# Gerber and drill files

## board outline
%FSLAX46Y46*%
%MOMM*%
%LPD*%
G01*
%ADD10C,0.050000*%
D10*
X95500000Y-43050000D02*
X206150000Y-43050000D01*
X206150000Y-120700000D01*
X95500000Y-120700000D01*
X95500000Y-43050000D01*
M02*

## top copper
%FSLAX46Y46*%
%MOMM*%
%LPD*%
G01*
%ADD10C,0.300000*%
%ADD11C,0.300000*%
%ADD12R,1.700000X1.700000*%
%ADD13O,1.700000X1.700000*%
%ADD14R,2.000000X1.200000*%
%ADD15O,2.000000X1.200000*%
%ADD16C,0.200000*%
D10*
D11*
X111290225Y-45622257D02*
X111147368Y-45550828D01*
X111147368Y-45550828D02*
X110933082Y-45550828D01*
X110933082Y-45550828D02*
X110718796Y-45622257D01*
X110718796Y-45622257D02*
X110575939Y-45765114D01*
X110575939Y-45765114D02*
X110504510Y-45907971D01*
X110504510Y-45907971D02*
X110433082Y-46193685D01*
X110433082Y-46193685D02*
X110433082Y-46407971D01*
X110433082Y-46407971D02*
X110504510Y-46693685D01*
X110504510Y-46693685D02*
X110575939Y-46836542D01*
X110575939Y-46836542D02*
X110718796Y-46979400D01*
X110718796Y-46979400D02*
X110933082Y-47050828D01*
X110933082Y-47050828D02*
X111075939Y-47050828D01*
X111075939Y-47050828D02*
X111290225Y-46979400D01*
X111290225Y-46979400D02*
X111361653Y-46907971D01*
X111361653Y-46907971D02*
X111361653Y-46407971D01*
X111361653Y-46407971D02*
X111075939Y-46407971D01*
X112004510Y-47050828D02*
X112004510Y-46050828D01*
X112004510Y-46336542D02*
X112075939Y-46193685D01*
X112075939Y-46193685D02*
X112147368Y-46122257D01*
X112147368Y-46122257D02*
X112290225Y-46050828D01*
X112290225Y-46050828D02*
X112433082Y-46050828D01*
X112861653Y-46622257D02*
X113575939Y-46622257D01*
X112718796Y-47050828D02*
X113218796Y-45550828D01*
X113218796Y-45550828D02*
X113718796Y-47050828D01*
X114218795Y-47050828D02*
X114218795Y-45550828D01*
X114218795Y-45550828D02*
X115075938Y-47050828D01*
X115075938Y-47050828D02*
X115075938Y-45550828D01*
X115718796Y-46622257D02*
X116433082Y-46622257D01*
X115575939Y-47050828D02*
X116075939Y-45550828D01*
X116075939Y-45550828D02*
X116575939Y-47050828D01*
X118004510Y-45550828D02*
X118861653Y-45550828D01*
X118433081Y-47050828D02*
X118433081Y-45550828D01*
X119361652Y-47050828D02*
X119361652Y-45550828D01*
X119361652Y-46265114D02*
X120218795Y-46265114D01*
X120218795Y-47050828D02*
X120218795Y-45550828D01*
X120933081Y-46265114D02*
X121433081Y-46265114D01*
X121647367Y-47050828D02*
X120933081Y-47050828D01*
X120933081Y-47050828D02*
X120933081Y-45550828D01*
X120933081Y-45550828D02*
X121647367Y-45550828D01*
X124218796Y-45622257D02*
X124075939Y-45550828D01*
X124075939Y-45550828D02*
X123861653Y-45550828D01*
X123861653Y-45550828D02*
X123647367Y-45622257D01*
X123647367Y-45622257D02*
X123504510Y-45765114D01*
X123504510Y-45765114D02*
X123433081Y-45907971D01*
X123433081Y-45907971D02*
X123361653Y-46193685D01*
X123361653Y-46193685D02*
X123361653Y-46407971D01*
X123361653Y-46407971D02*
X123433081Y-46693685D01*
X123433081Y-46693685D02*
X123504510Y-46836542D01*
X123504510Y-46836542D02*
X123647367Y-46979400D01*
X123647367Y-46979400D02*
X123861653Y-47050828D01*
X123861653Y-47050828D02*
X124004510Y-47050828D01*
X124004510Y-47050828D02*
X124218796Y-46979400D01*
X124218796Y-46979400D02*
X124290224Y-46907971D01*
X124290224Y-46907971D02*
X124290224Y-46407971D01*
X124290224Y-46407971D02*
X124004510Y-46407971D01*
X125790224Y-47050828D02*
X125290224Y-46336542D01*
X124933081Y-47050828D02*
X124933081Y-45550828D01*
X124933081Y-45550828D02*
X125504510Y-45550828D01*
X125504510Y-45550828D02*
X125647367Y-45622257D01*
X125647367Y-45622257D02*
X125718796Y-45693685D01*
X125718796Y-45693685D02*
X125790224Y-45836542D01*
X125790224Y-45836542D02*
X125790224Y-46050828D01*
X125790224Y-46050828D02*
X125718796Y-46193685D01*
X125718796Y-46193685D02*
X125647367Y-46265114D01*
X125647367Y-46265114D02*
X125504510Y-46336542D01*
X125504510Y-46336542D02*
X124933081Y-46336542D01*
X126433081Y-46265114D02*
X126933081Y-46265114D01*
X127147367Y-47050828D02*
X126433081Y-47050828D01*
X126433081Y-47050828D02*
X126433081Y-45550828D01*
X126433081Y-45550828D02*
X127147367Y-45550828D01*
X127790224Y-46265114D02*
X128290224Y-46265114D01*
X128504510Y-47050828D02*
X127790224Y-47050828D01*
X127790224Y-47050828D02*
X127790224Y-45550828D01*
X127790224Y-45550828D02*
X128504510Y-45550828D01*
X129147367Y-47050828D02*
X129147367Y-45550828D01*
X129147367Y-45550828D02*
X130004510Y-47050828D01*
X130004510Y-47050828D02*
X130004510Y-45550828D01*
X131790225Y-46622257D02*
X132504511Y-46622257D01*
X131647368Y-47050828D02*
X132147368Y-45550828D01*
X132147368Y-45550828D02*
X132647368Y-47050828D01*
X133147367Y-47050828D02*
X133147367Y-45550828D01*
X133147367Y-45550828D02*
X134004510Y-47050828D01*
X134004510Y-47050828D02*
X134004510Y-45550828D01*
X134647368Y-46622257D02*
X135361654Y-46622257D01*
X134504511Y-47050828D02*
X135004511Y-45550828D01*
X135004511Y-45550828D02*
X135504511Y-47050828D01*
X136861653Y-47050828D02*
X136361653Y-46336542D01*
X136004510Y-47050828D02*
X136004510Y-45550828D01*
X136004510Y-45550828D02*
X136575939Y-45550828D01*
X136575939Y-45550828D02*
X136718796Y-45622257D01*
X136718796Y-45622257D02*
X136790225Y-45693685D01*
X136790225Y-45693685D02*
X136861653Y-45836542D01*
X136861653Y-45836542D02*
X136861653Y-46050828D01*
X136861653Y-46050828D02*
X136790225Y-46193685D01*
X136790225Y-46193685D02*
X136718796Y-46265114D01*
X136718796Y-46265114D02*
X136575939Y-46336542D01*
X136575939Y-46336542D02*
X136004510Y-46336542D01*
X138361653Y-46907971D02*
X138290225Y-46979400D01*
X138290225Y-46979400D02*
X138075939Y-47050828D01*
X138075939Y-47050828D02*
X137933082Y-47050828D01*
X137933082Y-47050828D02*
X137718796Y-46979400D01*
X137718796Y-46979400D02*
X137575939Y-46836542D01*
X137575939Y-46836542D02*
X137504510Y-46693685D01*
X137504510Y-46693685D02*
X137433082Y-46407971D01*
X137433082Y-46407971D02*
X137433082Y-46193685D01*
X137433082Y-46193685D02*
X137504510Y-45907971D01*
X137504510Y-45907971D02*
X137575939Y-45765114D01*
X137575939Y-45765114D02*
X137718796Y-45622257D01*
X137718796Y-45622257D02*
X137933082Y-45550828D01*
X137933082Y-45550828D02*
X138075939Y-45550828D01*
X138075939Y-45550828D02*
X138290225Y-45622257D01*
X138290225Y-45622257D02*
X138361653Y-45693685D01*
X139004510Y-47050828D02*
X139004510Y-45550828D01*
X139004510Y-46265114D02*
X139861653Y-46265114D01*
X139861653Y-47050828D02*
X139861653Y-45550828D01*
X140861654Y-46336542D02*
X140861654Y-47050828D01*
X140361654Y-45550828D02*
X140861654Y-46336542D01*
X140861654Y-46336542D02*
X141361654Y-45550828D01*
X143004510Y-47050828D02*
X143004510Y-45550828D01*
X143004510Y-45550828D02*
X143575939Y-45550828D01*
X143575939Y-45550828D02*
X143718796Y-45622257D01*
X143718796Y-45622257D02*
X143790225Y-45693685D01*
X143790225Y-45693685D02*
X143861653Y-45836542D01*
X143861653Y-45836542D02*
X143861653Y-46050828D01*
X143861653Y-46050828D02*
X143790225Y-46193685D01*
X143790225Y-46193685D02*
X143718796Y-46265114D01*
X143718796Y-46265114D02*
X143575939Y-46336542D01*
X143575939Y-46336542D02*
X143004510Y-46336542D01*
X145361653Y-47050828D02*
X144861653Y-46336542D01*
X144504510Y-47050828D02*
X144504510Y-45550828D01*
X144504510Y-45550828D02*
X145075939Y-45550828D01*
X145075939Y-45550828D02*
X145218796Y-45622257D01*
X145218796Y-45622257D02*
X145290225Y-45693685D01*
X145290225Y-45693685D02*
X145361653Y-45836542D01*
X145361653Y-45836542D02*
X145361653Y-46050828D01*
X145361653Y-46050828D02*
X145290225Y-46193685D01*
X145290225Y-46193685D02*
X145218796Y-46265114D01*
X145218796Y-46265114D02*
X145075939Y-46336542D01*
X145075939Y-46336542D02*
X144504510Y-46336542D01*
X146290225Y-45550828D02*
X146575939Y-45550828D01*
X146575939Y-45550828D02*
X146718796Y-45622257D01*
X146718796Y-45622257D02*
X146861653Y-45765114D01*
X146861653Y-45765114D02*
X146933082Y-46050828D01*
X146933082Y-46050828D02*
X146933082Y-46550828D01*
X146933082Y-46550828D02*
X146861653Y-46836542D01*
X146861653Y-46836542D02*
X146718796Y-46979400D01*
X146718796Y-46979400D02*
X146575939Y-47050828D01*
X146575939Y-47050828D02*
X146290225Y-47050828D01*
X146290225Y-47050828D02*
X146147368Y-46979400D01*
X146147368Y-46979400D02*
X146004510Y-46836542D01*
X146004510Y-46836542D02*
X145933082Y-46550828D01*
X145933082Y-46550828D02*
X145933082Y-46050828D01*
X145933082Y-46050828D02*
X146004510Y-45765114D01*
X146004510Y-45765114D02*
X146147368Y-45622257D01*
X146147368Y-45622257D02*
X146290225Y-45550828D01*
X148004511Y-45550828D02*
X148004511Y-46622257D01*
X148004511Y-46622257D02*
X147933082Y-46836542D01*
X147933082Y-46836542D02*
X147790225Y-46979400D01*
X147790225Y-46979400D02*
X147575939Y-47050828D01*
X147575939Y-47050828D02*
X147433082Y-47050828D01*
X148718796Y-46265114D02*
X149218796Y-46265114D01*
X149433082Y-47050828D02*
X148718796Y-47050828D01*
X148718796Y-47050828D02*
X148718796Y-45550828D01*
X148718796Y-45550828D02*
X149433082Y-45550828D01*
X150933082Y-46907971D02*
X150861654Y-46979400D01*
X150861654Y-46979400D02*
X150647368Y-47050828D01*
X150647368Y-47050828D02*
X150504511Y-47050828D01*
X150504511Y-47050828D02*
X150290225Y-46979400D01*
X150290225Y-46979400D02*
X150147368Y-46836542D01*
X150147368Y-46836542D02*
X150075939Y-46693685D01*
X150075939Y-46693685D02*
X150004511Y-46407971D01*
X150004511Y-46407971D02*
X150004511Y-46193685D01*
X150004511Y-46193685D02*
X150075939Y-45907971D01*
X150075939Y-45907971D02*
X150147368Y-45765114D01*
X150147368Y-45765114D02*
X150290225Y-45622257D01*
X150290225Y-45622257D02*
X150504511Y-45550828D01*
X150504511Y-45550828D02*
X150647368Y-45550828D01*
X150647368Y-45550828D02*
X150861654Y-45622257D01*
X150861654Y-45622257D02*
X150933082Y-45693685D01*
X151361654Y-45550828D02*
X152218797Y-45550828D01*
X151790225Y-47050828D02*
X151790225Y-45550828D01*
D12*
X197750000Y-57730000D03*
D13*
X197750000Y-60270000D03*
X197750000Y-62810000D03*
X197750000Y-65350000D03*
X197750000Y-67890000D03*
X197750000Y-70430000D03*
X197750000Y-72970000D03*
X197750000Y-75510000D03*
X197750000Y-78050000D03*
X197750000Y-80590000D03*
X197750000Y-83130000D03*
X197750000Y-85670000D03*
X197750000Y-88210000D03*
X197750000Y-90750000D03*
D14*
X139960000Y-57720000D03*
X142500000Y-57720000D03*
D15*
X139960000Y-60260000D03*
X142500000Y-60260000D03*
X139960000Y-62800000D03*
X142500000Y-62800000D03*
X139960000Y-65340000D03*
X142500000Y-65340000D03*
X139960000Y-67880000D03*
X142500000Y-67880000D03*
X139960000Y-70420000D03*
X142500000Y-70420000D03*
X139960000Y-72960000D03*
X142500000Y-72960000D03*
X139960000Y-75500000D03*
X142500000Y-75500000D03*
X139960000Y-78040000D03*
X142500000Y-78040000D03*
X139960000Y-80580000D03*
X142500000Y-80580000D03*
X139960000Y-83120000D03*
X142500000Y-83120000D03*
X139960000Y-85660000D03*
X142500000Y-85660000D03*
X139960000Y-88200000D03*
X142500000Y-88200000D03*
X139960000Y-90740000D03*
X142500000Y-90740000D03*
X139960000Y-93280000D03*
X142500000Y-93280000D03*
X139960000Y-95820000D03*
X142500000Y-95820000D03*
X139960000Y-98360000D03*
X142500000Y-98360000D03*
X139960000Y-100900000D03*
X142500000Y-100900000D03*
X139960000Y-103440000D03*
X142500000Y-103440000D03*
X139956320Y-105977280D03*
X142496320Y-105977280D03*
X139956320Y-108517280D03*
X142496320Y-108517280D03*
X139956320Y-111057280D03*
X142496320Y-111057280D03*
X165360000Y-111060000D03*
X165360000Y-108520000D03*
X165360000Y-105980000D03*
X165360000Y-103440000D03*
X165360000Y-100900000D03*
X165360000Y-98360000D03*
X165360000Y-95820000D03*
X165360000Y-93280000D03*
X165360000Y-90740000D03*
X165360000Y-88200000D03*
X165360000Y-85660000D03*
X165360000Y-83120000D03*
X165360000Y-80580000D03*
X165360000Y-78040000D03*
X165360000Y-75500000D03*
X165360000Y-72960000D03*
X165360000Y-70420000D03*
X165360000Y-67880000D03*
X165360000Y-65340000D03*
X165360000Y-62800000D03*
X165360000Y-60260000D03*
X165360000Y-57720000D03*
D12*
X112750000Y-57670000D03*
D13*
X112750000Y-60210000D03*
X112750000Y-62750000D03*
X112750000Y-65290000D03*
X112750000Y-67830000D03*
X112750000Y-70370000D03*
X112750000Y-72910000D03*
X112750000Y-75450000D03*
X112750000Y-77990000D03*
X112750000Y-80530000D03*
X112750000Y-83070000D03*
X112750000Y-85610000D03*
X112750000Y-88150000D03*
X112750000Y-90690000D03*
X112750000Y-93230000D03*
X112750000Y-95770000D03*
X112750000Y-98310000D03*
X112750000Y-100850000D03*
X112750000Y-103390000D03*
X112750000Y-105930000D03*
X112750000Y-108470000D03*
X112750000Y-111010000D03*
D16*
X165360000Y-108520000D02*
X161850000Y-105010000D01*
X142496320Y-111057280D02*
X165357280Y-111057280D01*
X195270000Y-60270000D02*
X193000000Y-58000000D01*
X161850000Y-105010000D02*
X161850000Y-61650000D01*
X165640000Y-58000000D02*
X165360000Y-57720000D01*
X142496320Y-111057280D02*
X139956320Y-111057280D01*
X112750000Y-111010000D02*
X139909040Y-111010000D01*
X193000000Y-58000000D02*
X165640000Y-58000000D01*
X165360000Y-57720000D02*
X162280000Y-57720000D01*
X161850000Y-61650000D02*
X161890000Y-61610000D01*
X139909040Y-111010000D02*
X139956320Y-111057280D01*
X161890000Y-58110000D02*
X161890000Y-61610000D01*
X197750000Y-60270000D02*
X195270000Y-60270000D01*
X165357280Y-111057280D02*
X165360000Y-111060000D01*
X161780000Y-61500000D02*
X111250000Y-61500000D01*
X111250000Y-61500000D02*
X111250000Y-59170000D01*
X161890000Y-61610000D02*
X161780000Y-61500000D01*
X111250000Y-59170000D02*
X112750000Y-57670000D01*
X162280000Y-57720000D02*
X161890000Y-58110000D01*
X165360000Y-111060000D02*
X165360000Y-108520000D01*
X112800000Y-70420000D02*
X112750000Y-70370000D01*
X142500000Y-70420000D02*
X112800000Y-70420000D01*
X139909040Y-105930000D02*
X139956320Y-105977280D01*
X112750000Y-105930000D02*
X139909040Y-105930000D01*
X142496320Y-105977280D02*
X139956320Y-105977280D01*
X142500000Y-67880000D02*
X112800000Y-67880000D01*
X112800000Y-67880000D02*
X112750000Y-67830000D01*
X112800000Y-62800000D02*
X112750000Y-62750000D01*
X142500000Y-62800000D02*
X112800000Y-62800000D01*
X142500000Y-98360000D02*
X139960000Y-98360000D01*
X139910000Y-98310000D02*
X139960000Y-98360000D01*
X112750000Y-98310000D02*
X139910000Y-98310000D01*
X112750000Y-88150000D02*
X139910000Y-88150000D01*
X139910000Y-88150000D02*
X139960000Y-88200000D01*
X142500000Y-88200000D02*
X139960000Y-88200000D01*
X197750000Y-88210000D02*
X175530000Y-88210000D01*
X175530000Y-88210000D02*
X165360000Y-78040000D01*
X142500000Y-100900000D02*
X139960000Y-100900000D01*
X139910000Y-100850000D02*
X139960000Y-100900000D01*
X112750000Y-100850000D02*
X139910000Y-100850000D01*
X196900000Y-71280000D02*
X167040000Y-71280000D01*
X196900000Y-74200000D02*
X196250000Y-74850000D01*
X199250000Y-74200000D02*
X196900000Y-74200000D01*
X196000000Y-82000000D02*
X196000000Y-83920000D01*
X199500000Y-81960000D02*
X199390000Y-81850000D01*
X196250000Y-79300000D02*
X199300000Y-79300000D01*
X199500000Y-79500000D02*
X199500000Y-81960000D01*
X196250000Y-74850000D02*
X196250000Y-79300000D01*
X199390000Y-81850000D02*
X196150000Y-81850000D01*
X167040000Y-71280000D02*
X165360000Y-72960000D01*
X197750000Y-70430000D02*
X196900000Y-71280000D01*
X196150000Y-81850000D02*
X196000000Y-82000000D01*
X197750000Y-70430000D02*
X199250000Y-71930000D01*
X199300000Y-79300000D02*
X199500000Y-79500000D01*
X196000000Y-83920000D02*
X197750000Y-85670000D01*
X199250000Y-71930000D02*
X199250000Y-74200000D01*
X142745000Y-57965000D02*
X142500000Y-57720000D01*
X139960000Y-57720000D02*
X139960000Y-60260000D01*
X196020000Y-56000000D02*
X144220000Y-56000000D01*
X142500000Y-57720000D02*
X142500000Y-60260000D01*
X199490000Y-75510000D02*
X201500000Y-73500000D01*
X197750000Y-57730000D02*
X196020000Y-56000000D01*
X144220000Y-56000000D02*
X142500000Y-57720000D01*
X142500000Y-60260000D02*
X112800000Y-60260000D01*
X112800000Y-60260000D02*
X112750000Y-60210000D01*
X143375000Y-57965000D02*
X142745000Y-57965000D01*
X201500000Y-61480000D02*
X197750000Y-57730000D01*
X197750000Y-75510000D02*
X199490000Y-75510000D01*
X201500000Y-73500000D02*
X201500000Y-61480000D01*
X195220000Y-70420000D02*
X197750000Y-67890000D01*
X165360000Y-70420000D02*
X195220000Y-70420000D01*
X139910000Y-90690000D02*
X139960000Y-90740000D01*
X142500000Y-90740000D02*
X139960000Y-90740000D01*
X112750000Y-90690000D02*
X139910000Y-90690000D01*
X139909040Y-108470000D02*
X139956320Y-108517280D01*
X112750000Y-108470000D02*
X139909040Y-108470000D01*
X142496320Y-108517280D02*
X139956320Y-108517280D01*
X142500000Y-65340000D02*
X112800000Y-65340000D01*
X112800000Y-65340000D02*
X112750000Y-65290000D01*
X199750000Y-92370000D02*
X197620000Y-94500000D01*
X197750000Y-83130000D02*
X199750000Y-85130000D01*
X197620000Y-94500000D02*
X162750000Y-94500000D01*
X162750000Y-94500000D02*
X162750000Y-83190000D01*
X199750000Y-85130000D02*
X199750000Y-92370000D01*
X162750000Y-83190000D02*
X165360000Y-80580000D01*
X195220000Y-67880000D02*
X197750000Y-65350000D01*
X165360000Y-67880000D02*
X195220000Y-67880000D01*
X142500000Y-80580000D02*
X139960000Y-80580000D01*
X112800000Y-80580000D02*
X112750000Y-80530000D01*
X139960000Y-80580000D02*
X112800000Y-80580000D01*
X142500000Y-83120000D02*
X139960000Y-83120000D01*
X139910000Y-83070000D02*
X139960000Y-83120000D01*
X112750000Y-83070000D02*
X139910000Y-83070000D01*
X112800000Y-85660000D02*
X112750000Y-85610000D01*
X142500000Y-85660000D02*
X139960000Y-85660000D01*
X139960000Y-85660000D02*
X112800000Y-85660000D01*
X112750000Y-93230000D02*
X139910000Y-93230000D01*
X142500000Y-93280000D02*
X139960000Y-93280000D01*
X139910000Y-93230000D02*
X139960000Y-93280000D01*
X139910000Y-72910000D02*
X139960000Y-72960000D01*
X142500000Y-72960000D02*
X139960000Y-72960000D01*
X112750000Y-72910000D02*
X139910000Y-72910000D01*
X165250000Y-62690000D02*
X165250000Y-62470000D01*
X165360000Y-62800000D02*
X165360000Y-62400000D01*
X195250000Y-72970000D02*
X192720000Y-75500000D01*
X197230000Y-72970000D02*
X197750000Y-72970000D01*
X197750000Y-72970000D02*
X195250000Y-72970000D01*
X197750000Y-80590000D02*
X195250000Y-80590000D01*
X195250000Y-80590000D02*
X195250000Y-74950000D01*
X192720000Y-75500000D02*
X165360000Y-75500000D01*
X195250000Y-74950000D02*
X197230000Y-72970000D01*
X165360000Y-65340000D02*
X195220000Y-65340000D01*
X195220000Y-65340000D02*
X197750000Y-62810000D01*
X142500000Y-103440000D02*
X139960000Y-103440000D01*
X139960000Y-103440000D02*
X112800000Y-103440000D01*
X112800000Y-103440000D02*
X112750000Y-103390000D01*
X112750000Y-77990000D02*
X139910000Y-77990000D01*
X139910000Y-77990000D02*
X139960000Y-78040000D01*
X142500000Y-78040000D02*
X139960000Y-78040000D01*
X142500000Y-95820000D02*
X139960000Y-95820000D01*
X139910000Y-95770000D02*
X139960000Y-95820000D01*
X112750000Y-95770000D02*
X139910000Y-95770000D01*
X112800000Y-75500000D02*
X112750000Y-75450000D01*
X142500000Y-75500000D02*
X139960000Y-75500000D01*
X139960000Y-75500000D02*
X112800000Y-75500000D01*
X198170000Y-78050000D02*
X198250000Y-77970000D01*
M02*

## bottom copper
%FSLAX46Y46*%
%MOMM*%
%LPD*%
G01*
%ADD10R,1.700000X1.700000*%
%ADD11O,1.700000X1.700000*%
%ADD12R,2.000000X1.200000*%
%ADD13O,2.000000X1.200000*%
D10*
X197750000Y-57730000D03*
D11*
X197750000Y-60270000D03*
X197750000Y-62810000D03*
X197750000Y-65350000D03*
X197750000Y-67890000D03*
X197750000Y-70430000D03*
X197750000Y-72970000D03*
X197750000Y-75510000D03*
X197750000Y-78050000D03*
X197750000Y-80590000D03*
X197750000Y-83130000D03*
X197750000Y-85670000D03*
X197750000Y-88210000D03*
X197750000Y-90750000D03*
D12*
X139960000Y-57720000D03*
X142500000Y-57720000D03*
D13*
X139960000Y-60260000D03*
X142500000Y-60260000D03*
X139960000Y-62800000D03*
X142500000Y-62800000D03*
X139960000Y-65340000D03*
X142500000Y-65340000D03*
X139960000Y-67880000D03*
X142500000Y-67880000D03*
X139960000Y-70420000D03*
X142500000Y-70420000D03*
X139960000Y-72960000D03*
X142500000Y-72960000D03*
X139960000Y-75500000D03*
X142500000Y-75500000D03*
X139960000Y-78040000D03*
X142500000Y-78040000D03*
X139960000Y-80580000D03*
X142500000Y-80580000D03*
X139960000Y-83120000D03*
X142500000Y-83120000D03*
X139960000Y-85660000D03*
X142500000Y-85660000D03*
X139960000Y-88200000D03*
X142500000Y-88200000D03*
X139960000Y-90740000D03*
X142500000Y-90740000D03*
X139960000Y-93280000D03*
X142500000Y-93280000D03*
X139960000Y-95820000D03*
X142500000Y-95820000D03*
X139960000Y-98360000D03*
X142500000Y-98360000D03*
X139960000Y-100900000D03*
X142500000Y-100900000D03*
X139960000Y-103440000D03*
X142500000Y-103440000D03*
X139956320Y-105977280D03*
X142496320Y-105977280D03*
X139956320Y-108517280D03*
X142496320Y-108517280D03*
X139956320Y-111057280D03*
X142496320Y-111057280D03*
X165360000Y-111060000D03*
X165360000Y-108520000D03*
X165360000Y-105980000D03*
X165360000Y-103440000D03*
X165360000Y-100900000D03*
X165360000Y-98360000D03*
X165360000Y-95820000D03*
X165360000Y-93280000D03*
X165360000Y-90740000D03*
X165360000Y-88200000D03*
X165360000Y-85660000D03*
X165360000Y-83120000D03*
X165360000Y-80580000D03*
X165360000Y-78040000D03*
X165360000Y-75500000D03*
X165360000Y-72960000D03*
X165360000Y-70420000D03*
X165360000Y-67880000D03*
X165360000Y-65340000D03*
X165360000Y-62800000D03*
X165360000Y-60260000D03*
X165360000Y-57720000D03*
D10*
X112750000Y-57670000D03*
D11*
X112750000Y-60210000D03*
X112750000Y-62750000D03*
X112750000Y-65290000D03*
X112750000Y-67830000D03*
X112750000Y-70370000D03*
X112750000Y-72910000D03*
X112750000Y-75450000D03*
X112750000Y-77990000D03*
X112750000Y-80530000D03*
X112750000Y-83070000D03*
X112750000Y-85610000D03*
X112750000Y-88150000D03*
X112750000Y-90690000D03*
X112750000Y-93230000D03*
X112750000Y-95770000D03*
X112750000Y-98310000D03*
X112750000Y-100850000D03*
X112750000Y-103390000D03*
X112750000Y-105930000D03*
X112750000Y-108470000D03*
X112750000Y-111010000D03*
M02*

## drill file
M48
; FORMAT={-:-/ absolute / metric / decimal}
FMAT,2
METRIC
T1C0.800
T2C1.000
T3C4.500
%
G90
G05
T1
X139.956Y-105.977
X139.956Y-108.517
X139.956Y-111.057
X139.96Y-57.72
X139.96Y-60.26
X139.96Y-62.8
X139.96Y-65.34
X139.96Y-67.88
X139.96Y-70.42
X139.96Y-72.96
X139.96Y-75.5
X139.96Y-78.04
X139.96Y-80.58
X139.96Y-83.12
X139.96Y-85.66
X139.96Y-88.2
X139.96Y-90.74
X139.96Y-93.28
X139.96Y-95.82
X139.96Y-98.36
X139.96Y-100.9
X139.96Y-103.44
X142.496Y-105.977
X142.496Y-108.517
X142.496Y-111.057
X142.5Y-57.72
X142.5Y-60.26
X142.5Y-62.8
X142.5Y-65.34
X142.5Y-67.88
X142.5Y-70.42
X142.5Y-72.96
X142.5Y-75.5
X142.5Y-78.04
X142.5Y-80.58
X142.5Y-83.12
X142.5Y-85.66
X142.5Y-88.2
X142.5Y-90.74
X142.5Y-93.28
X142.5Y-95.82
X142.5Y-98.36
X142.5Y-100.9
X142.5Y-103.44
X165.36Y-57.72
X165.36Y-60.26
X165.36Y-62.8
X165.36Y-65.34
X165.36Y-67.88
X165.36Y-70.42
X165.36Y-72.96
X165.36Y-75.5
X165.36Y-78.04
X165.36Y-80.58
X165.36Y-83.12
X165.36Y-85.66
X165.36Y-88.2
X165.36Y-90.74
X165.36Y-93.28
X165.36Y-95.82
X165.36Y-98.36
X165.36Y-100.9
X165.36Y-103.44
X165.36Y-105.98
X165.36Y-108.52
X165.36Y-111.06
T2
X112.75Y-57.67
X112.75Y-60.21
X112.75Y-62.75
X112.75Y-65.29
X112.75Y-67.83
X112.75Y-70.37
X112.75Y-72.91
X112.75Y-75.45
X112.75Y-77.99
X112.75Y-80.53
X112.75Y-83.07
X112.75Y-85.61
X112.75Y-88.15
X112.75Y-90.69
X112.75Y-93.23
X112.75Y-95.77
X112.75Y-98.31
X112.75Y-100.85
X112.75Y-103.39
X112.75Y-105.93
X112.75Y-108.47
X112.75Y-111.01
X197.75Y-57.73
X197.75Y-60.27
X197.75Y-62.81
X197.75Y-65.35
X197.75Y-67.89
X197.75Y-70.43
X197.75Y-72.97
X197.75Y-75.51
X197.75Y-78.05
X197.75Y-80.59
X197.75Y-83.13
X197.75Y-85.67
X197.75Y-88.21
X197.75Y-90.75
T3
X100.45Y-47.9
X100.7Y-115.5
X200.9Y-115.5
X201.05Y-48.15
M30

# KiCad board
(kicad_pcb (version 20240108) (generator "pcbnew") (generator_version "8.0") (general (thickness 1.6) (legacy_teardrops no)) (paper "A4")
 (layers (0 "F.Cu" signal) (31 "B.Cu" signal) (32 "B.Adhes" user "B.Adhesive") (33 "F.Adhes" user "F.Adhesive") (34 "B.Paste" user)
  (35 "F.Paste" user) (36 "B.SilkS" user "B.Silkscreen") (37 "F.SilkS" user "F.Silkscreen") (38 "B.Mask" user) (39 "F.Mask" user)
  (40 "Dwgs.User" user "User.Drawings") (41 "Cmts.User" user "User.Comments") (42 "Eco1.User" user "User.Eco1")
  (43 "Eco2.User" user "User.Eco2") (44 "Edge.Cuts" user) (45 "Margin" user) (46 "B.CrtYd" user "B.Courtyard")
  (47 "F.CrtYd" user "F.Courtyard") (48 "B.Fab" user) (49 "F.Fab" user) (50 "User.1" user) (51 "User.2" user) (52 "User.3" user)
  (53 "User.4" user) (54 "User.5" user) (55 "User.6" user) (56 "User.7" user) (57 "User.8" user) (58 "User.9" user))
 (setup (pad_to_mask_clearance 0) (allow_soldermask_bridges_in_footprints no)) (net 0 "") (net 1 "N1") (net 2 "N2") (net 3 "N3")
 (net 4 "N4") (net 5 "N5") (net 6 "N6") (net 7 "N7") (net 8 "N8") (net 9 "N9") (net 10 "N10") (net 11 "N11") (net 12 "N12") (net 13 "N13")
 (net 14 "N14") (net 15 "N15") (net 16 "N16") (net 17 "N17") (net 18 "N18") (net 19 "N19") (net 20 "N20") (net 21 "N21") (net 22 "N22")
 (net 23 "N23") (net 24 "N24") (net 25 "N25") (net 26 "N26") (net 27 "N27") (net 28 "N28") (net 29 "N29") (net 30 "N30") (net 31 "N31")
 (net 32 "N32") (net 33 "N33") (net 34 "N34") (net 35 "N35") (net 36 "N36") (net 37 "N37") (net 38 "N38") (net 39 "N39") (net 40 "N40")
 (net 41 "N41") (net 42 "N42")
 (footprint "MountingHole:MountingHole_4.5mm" (layer "F.Cu") (at 100.7 115.5)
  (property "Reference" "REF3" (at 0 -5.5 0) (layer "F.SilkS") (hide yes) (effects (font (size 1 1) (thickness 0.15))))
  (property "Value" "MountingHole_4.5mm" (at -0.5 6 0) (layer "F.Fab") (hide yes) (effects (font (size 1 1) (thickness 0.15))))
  (pad "" np_thru_hole circle (at 0 0) (size 4.5 4.5) (drill 4.5) (layers "*.Cu" "*.Mask")))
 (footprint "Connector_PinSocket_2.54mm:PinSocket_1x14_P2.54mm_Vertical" (layer "F.Cu") (at 197.75 57.73)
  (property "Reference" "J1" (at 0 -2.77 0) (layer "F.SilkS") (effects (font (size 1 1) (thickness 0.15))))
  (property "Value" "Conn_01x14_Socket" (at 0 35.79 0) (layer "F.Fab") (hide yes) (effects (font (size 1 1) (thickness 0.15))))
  (pad "1" thru_hole rect (at 0 0) (size 1.7 1.7) (drill 1) (layers "*.Cu" "*.Mask") (remove_unused_layers no) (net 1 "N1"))
  (pad "2" thru_hole oval (at 0 2.54) (size 1.7 1.7) (drill 1) (layers "*.Cu" "*.Mask") (remove_unused_layers no) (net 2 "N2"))
  (pad "3" thru_hole oval (at 0 5.08) (size 1.7 1.7) (drill 1) (layers "*.Cu" "*.Mask") (remove_unused_layers no) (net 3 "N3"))
  (pad "4" thru_hole oval (at 0 7.62) (size 1.7 1.7) (drill 1) (layers "*.Cu" "*.Mask") (remove_unused_layers no) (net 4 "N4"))
  (pad "5" thru_hole oval (at 0 10.16) (size 1.7 1.7) (drill 1) (layers "*.Cu" "*.Mask") (remove_unused_layers no) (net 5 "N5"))
  (pad "6" thru_hole oval (at 0 12.7) (size 1.7 1.7) (drill 1) (layers "*.Cu" "*.Mask") (remove_unused_layers no) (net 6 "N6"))
  (pad "7" thru_hole oval (at 0 15.24) (size 1.7 1.7) (drill 1) (layers "*.Cu" "*.Mask") (remove_unused_layers no) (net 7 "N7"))
  (pad "8" thru_hole oval (at 0 17.78) (size 1.7 1.7) (drill 1) (layers "*.Cu" "*.Mask") (remove_unused_layers no) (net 1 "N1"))
  (pad "9" thru_hole oval (at 0 20.32) (size 1.7 1.7) (drill 1) (layers "*.Cu" "*.Mask") (remove_unused_layers no) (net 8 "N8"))
  (pad "10" thru_hole oval (at 0 22.86) (size 1.7 1.7) (drill 1) (layers "*.Cu" "*.Mask") (remove_unused_layers no) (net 7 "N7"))
  (pad "11" thru_hole oval (at 0 25.4) (size 1.7 1.7) (drill 1) (layers "*.Cu" "*.Mask") (remove_unused_layers no) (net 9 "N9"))
  (pad "12" thru_hole oval (at 0 27.94) (size 1.7 1.7) (drill 1) (layers "*.Cu" "*.Mask") (remove_unused_layers no) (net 6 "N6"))
  (pad "13" thru_hole oval (at 0 30.48) (size 1.7 1.7) (drill 1) (layers "*.Cu" "*.Mask") (remove_unused_layers no) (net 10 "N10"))
  (pad "14" thru_hole oval (at 0 33.02) (size 1.7 1.7) (drill 1) (layers "*.Cu" "*.Mask") (remove_unused_layers no) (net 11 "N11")))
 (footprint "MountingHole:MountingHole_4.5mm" (layer "F.Cu") (at 100.45 47.9)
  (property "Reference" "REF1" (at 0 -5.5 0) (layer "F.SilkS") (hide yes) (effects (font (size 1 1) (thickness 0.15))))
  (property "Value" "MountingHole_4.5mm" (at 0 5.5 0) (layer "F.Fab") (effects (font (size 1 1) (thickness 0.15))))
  (pad "" np_thru_hole circle (at 0 0) (size 4.5 4.5) (drill 4.5) (layers "*.Cu" "*.Mask")))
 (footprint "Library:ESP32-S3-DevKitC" (layer "F.Cu") (at 163.25 68.97)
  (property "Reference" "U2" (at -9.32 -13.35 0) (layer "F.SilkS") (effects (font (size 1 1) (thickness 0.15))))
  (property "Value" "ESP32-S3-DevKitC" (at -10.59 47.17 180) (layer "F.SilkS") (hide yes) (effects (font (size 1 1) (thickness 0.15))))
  (pad "1" thru_hole rect (at -23.29 -11.25 270) (size 1.2 2) (drill 0.8) (layers "*.Cu" "*.Mask") (remove_unused_layers no) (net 1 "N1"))
  (pad "1" thru_hole rect (at -20.75 -11.25 270) (size 1.2 2) (drill 0.8) (layers "*.Cu" "*.Mask") (remove_unused_layers no) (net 1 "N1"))
  (pad "2" thru_hole oval (at -23.29 -8.71 270) (size 1.2 2) (drill 0.8) (layers "*.Cu" "*.Mask") (remove_unused_layers no) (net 1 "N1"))
  (pad "2" thru_hole oval (at -20.75 -8.71 270) (size 1.2 2) (drill 0.8) (layers "*.Cu" "*.Mask") (remove_unused_layers no) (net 1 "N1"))
  (pad "3" thru_hole oval (at -23.29 -6.17 270) (size 1.2 2) (drill 0.8) (layers "*.Cu" "*.Mask") (remove_unused_layers no) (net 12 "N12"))
  (pad "3" thru_hole oval (at -20.75 -6.17 270) (size 1.2 2) (drill 0.8) (layers "*.Cu" "*.Mask") (remove_unused_layers no) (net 12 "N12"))
  (pad "4" thru_hole oval (at -23.29 -3.63 270) (size 1.2 2) (drill 0.8) (layers "*.Cu" "*.Mask") (remove_unused_layers no) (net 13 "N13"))
  (pad "4" thru_hole oval (at -20.75 -3.63 270) (size 1.2 2) (drill 0.8) (layers "*.Cu" "*.Mask") (remove_unused_layers no) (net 13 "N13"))
  (pad "5" thru_hole oval (at -23.29 -1.09 270) (size 1.2 2) (drill 0.8) (layers "*.Cu" "*.Mask") (remove_unused_layers no) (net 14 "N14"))
  (pad "5" thru_hole oval (at -20.75 -1.09 270) (size 1.2 2) (drill 0.8) (layers "*.Cu" "*.Mask") (remove_unused_layers no) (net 14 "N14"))
  (pad "6" thru_hole oval (at -23.29 1.45 270) (size 1.2 2) (drill 0.8) (layers "*.Cu" "*.Mask") (remove_unused_layers no) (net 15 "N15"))
  (pad "6" thru_hole oval (at -20.75 1.45 270) (size 1.2 2) (drill 0.8) (layers "*.Cu" "*.Mask") (remove_unused_layers no) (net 15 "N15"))
  (pad "7" thru_hole oval (at -23.29 3.99 270) (size 1.2 2) (drill 0.8) (layers "*.Cu" "*.Mask") (remove_unused_layers no) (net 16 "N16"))
  (pad "7" thru_hole oval (at -20.75 3.99 270) (size 1.2 2) (drill 0.8) (layers "*.Cu" "*.Mask") (remove_unused_layers no) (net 16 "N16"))
  (pad "8" thru_hole oval (at -23.29 6.53 270) (size 1.2 2) (drill 0.8) (layers "*.Cu" "*.Mask") (remove_unused_layers no) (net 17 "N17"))
  (pad "8" thru_hole oval (at -20.75 6.53 270) (size 1.2 2) (drill 0.8) (layers "*.Cu" "*.Mask") (remove_unused_layers no) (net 17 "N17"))
  (pad "9" thru_hole oval (at -23.29 9.07 270) (size 1.2 2) (drill 0.8) (layers "*.Cu" "*.Mask") (remove_unused_layers no) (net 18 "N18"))
  (pad "9" thru_hole oval (at -20.75 9.07 270) (size 1.2 2) (drill 0.8) (layers "*.Cu" "*.Mask") (remove_unused_layers no) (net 18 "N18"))
  (pad "10" thru_hole oval (at -23.29 11.61 270) (size 1.2 2) (drill 0.8) (layers "*.Cu" "*.Mask") (remove_unused_layers no) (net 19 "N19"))
  (pad "10" thru_hole oval (at -20.75 11.61 270) (size 1.2 2) (drill 0.8) (layers "*.Cu" "*.Mask") (remove_unused_layers no) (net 19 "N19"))
  (pad "11" thru_hole oval (at -23.29 14.15 270) (size 1.2 2) (drill 0.8) (layers "*.Cu" "*.Mask") (remove_unused_layers no) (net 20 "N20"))
  (pad "11" thru_hole oval (at -20.75 14.15 270) (size 1.2 2) (drill 0.8) (layers "*.Cu" "*.Mask") (remove_unused_layers no) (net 20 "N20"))
  (pad "12" thru_hole oval (at -23.29 16.69 270) (size 1.2 2) (drill 0.8) (layers "*.Cu" "*.Mask") (remove_unused_layers no) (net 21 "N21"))
  (pad "12" thru_hole oval (at -20.75 16.69 270) (size 1.2 2) (drill 0.8) (layers "*.Cu" "*.Mask") (remove_unused_layers no) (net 21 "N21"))
  (pad "13" thru_hole oval (at -23.29 19.23 270) (size 1.2 2) (drill 0.8) (layers "*.Cu" "*.Mask") (remove_unused_layers no) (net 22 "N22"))
  (pad "13" thru_hole oval (at -20.75 19.23 270) (size 1.2 2) (drill 0.8) (layers "*.Cu" "*.Mask") (remove_unused_layers no) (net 22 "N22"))
  (pad "14" thru_hole oval (at -23.29 21.77 270) (size 1.2 2) (drill 0.8) (layers "*.Cu" "*.Mask") (remove_unused_layers no) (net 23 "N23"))
  (pad "14" thru_hole oval (at -20.75 21.77 270) (size 1.2 2) (drill 0.8) (layers "*.Cu" "*.Mask") (remove_unused_layers no) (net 23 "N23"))
  (pad "15" thru_hole oval (at -23.29 24.31 270) (size 1.2 2) (drill 0.8) (layers "*.Cu" "*.Mask") (remove_unused_layers no) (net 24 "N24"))
  (pad "15" thru_hole oval (at -20.75 24.31 270) (size 1.2 2) (drill 0.8) (layers "*.Cu" "*.Mask") (remove_unused_layers no) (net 24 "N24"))
  (pad "16" thru_hole oval (at -23.29 26.85 270) (size 1.2 2) (drill 0.8) (layers "*.Cu" "*.Mask") (remove_unused_layers no) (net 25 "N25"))
  (pad "16" thru_hole oval (at -20.75 26.85 270) (size 1.2 2) (drill 0.8) (layers "*.Cu" "*.Mask") (remove_unused_layers no) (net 25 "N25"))
  (pad "17" thru_hole oval (at -23.29 29.39 270) (size 1.2 2) (drill 0.8) (layers "*.Cu" "*.Mask") (remove_unused_layers no) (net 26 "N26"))
  (pad "17" thru_hole oval (at -20.75 29.39 270) (size 1.2 2) (drill 0.8) (layers "*.Cu" "*.Mask") (remove_unused_layers no) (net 26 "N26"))
  (pad "18" thru_hole oval (at -23.29 31.93 270) (size 1.2 2) (drill 0.8) (layers "*.Cu" "*.Mask") (remove_unused_layers no) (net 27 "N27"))
  (pad "18" thru_hole oval (at -20.75 31.93 270) (size 1.2 2) (drill 0.8) (layers "*.Cu" "*.Mask") (remove_unused_layers no) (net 27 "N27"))
  (pad "19" thru_hole oval (at -23.29 34.47 270) (size 1.2 2) (drill 0.8) (layers "*.Cu" "*.Mask") (remove_unused_layers no) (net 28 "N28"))
  (pad "19" thru_hole oval (at -20.75 34.47 270) (size 1.2 2) (drill 0.8) (layers "*.Cu" "*.Mask") (remove_unused_layers no) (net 28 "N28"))
  (pad "20" thru_hole oval (at -23.29368 37.00728 270) (size 1.2 2) (drill 0.8) (layers "*.Cu" "*.Mask") (remove_unused_layers no)
   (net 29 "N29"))
  (pad "20" thru_hole oval (at -20.75368 37.00728 270) (size 1.2 2) (drill 0.8) (layers "*.Cu" "*.Mask") (remove_unused_layers no)
   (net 29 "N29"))
  (pad "21" thru_hole oval (at -23.29368 39.54728 270) (size 1.2 2) (drill 0.8) (layers "*.Cu" "*.Mask") (remove_unused_layers no)
   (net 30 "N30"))
  (pad "21" thru_hole oval (at -20.75368 39.54728 270) (size 1.2 2) (drill 0.8) (layers "*.Cu" "*.Mask") (remove_unused_layers no)
   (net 30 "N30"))
  (pad "22" thru_hole oval (at -23.29368 42.08728 270) (size 1.2 2) (drill 0.8) (layers "*.Cu" "*.Mask") (remove_unused_layers no)
   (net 2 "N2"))
  (pad "22" thru_hole oval (at -20.75368 42.08728 270) (size 1.2 2) (drill 0.8) (layers "*.Cu" "*.Mask") (remove_unused_layers no)
   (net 2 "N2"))
  (pad "23" thru_hole oval (at 2.11 42.09 270) (size 1.2 2) (drill 0.8) (layers "*.Cu" "*.Mask") (remove_unused_layers no) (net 2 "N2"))
  (pad "24" thru_hole oval (at 2.11 39.55 270) (size 1.2 2) (drill 0.8) (layers "*.Cu" "*.Mask") (remove_unused_layers no) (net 2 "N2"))
  (pad "25" thru_hole oval (at 2.11 37.01 270) (size 1.2 2) (drill 0.8) (layers "*.Cu" "*.Mask") (remove_unused_layers no) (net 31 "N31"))
  (pad "26" thru_hole oval (at 2.11 34.47 270) (size 1.2 2) (drill 0.8) (layers "*.Cu" "*.Mask") (remove_unused_layers no) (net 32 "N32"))
  (pad "27" thru_hole oval (at 2.11 31.93 270) (size 1.2 2) (drill 0.8) (layers "*.Cu" "*.Mask") (remove_unused_layers no) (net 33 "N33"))
  (pad "28" thru_hole oval (at 2.11 29.39 270) (size 1.2 2) (drill 0.8) (layers "*.Cu" "*.Mask") (remove_unused_layers no) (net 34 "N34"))
  (pad "29" thru_hole oval (at 2.11 26.85 270) (size 1.2 2) (drill 0.8) (layers "*.Cu" "*.Mask") (remove_unused_layers no) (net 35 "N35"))
  (pad "30" thru_hole oval (at 2.11 24.31 270) (size 1.2 2) (drill 0.8) (layers "*.Cu" "*.Mask") (remove_unused_layers no) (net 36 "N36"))
  (pad "31" thru_hole oval (at 2.11 21.77 270) (size 1.2 2) (drill 0.8) (layers "*.Cu" "*.Mask") (remove_unused_layers no) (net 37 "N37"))
  (pad "32" thru_hole oval (at 2.11 19.23 270) (size 1.2 2) (drill 0.8) (layers "*.Cu" "*.Mask") (remove_unused_layers no) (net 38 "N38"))
  (pad "33" thru_hole oval (at 2.11 16.69 270) (size 1.2 2) (drill 0.8) (layers "*.Cu" "*.Mask") (remove_unused_layers no) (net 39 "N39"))
  (pad "34" thru_hole oval (at 2.11 14.15 270) (size 1.2 2) (drill 0.8) (layers "*.Cu" "*.Mask") (remove_unused_layers no) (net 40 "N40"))
  (pad "35" thru_hole oval (at 2.11 11.61 270) (size 1.2 2) (drill 0.8) (layers "*.Cu" "*.Mask") (remove_unused_layers no) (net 9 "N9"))
  (pad "36" thru_hole oval (at 2.11 9.07 270) (size 1.2 2) (drill 0.8) (layers "*.Cu" "*.Mask") (remove_unused_layers no) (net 10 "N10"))
  (pad "37" thru_hole oval (at 2.11 6.53 270) (size 1.2 2) (drill 0.8) (layers "*.Cu" "*.Mask") (remove_unused_layers no) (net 7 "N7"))
  (pad "38" thru_hole oval (at 2.11 3.99 270) (size 1.2 2) (drill 0.8) (layers "*.Cu" "*.Mask") (remove_unused_layers no) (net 6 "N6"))
  (pad "39" thru_hole oval (at 2.11 1.45 270) (size 1.2 2) (drill 0.8) (layers "*.Cu" "*.Mask") (remove_unused_layers no) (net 5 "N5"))
  (pad "40" thru_hole oval (at 2.11 -1.09 270) (size 1.2 2) (drill 0.8) (layers "*.Cu" "*.Mask") (remove_unused_layers no) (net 4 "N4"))
  (pad "41" thru_hole oval (at 2.11 -3.63 270) (size 1.2 2) (drill 0.8) (layers "*.Cu" "*.Mask") (remove_unused_layers no) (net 3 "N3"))
  (pad "42" thru_hole oval (at 2.11 -6.17 270) (size 1.2 2) (drill 0.8) (layers "*.Cu" "*.Mask") (remove_unused_layers no) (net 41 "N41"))
  (pad "43" thru_hole oval (at 2.11 -8.71 270) (size 1.2 2) (drill 0.8) (layers "*.Cu" "*.Mask") (remove_unused_layers no) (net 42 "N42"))
  (pad "44" thru_hole oval (at 2.11 -11.25 270) (size 1.2 2) (drill 0.8) (layers "*.Cu" "*.Mask") (remove_unused_layers no) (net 2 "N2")))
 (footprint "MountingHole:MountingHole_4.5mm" (layer "F.Cu") (at 200.9 115.5)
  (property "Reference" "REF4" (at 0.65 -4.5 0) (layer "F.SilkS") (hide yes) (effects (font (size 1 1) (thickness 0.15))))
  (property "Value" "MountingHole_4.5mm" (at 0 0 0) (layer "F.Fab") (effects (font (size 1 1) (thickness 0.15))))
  (pad "" np_thru_hole circle (at 0 0) (size 4.5 4.5) (drill 4.5) (layers "*.Cu" "*.Mask")))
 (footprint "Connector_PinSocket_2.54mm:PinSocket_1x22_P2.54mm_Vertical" (layer "F.Cu") (at 112.75 57.67)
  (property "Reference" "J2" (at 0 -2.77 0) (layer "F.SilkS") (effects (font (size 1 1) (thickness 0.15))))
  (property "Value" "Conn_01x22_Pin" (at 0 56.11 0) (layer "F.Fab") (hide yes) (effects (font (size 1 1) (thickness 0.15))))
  (pad "1" thru_hole rect (at 0 0) (size 1.7 1.7) (drill 1) (layers "*.Cu" "*.Mask") (remove_unused_layers no) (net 2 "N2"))
  (pad "2" thru_hole oval (at 0 2.54) (size 1.7 1.7) (drill 1) (layers "*.Cu" "*.Mask") (remove_unused_layers no) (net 1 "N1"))
  (pad "3" thru_hole oval (at 0 5.08) (size 1.7 1.7) (drill 1) (layers "*.Cu" "*.Mask") (remove_unused_layers no) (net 12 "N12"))
  (pad "4" thru_hole oval (at 0 7.62) (size 1.7 1.7) (drill 1) (layers "*.Cu" "*.Mask") (remove_unused_layers no) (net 13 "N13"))
  (pad "5" thru_hole oval (at 0 10.16) (size 1.7 1.7) (drill 1) (layers "*.Cu" "*.Mask") (remove_unused_layers no) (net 14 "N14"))
  (pad "6" thru_hole oval (at 0 12.7) (size 1.7 1.7) (drill 1) (layers "*.Cu" "*.Mask") (remove_unused_layers no) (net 15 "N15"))
  (pad "7" thru_hole oval (at 0 15.24) (size 1.7 1.7) (drill 1) (layers "*.Cu" "*.Mask") (remove_unused_layers no) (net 16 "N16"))
  (pad "8" thru_hole oval (at 0 17.78) (size 1.7 1.7) (drill 1) (layers "*.Cu" "*.Mask") (remove_unused_layers no) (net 17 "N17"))
  (pad "9" thru_hole oval (at 0 20.32) (size 1.7 1.7) (drill 1) (layers "*.Cu" "*.Mask") (remove_unused_layers no) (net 18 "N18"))
  (pad "10" thru_hole oval (at 0 22.86) (size 1.7 1.7) (drill 1) (layers "*.Cu" "*.Mask") (remove_unused_layers no) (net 19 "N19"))
  (pad "11" thru_hole oval (at 0 25.4) (size 1.7 1.7) (drill 1) (layers "*.Cu" "*.Mask") (remove_unused_layers no) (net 20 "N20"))
  (pad "12" thru_hole oval (at 0 27.94) (size 1.7 1.7) (drill 1) (layers "*.Cu" "*.Mask") (remove_unused_layers no) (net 21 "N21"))
  (pad "13" thru_hole oval (at 0 30.48) (size 1.7 1.7) (drill 1) (layers "*.Cu" "*.Mask") (remove_unused_layers no) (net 22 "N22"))
  (pad "14" thru_hole oval (at 0 33.02) (size 1.7 1.7) (drill 1) (layers "*.Cu" "*.Mask") (remove_unused_layers no) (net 23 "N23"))
  (pad "15" thru_hole oval (at 0 35.56) (size 1.7 1.7) (drill 1) (layers "*.Cu" "*.Mask") (remove_unused_layers no) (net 24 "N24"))
  (pad "16" thru_hole oval (at 0 38.1) (size 1.7 1.7) (drill 1) (layers "*.Cu" "*.Mask") (remove_unused_layers no) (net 25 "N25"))
  (pad "17" thru_hole oval (at 0 40.64) (size 1.7 1.7) (drill 1) (layers "*.Cu" "*.Mask") (remove_unused_layers no) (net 26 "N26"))
  (pad "18" thru_hole oval (at 0 43.18) (size 1.7 1.7) (drill 1) (layers "*.Cu" "*.Mask") (remove_unused_layers no) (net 27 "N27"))
  (pad "19" thru_hole oval (at 0 45.72) (size 1.7 1.7) (drill 1) (layers "*.Cu" "*.Mask") (remove_unused_layers no) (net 28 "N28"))
  (pad "20" thru_hole oval (at 0 48.26) (size 1.7 1.7) (drill 1) (layers "*.Cu" "*.Mask") (remove_unused_layers no) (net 29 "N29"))
  (pad "21" thru_hole oval (at 0 50.8) (size 1.7 1.7) (drill 1) (layers "*.Cu" "*.Mask") (remove_unused_layers no) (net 30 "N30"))
  (pad "22" thru_hole oval (at 0 53.34) (size 1.7 1.7) (drill 1) (layers "*.Cu" "*.Mask") (remove_unused_layers no) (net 2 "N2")))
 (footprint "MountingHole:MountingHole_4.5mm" (layer "F.Cu") (at 201.05 48.15)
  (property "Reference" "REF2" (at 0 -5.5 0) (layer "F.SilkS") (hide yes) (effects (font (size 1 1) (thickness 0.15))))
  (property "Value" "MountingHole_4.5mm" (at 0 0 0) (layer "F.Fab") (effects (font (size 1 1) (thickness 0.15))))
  (pad "" np_thru_hole circle (at 0 0) (size 4.5 4.5) (drill 4.5) (layers "*.Cu" "*.Mask")))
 (gr_rect (start 95.5 43.05) (end 206.15 120.7) (stroke (width 0.05) (type default)) (fill none) (layer "Edge.Cuts"))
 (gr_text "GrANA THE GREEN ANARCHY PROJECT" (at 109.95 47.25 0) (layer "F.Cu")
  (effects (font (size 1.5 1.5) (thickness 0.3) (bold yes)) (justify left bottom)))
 (segment (start 165.36 108.52) (end 161.85 105.01) (width 0.2) (layer "F.Cu") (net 2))
 (segment (start 142.49632 111.05728) (end 165.35728 111.05728) (width 0.2) (layer "F.Cu") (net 2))
 (segment (start 195.27 60.27) (end 193 58) (width 0.2) (layer "F.Cu") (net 2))
 (segment (start 161.85 105.01) (end 161.85 61.65) (width 0.2) (layer "F.Cu") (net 2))
 (segment (start 165.64 58) (end 165.36 57.72) (width 0.2) (layer "F.Cu") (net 2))
 (segment (start 142.49632 111.05728) (end 139.95632 111.05728) (width 0.2) (layer "F.Cu") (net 2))
 (segment (start 112.75 111.01) (end 139.90904 111.01) (width 0.2) (layer "F.Cu") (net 2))
 (segment (start 193 58) (end 165.64 58) (width 0.2) (layer "F.Cu") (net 2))
 (segment (start 165.36 57.72) (end 162.28 57.72) (width 0.2) (layer "F.Cu") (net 2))
 (segment (start 161.85 61.65) (end 161.89 61.61) (width 0.2) (layer "F.Cu") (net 2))
 (segment (start 139.90904 111.01) (end 139.95632 111.05728) (width 0.2) (layer "F.Cu") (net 2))
 (segment (start 161.89 58.11) (end 161.89 61.61) (width 0.2) (layer "F.Cu") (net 2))
 (segment (start 197.75 60.27) (end 195.27 60.27) (width 0.2) (layer "F.Cu") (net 2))
 (segment (start 165.35728 111.05728) (end 165.36 111.06) (width 0.2) (layer "F.Cu") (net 2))
 (segment (start 161.78 61.5) (end 111.25 61.5) (width 0.2) (layer "F.Cu") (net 2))
 (segment (start 111.25 61.5) (end 111.25 59.17) (width 0.2) (layer "F.Cu") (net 2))
 (segment (start 161.89 61.61) (end 161.78 61.5) (width 0.2) (layer "F.Cu") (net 2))
 (segment (start 111.25 59.17) (end 112.75 57.67) (width 0.2) (layer "F.Cu") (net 2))
 (segment (start 162.28 57.72) (end 161.89 58.11) (width 0.2) (layer "F.Cu") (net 2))
 (segment (start 165.36 111.06) (end 165.36 108.52) (width 0.2) (layer "F.Cu") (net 2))
 (segment (start 112.8 70.42) (end 112.75 70.37) (width 0.2) (layer "F.Cu") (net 15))
 (segment (start 142.5 70.42) (end 112.8 70.42) (width 0.2) (layer "F.Cu") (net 15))
 (segment (start 139.90904 105.93) (end 139.95632 105.97728) (width 0.2) (layer "F.Cu") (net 29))
 (segment (start 112.75 105.93) (end 139.90904 105.93) (width 0.2) (layer "F.Cu") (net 29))
 (segment (start 142.49632 105.97728) (end 139.95632 105.97728) (width 0.2) (layer "F.Cu") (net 29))
 (segment (start 142.5 67.88) (end 112.8 67.88) (width 0.2) (layer "F.Cu") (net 14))
 (segment (start 112.8 67.88) (end 112.75 67.83) (width 0.2) (layer "F.Cu") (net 14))
 (segment (start 112.8 62.8) (end 112.75 62.75) (width 0.2) (layer "F.Cu") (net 12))
 (segment (start 142.5 62.8) (end 112.8 62.8) (width 0.2) (layer "F.Cu") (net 12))
 (segment (start 142.5 98.36) (end 139.96 98.36) (width 0.2) (layer "F.Cu") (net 26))
 (segment (start 139.91 98.31) (end 139.96 98.36) (width 0.2) (layer "F.Cu") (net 26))
 (segment (start 112.75 98.31) (end 139.91 98.31) (width 0.2) (layer "F.Cu") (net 26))
 (segment (start 112.75 88.15) (end 139.91 88.15) (width 0.2) (layer "F.Cu") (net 22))
 (segment (start 139.91 88.15) (end 139.96 88.2) (width 0.2) (layer "F.Cu") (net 22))
 (segment (start 142.5 88.2) (end 139.96 88.2) (width 0.2) (layer "F.Cu") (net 22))
 (segment (start 197.75 88.21) (end 175.53 88.21) (width 0.2) (layer "F.Cu") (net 10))
 (segment (start 175.53 88.21) (end 165.36 78.04) (width 0.2) (layer "F.Cu") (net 10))
 (segment (start 142.5 100.9) (end 139.96 100.9) (width 0.2) (layer "F.Cu") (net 27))
 (segment (start 139.91 100.85) (end 139.96 100.9) (width 0.2) (layer "F.Cu") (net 27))
 (segment (start 112.75 100.85) (end 139.91 100.85) (width 0.2) (layer "F.Cu") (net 27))
 (segment (start 196.9 71.28) (end 167.04 71.28) (width 0.2) (layer "F.Cu") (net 6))
 (segment (start 196.9 74.2) (end 196.25 74.85) (width 0.2) (layer "F.Cu") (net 6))
 (segment (start 199.25 74.2) (end 196.9 74.2) (width 0.2) (layer "F.Cu") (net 6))
 (segment (start 196 82) (end 196 83.92) (width 0.2) (layer "F.Cu") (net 6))
 (segment (start 199.5 81.96) (end 199.39 81.85) (width 0.2) (layer "F.Cu") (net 6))
 (segment (start 196.25 79.3) (end 199.3 79.3) (width 0.2) (layer "F.Cu") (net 6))
 (segment (start 199.5 79.5) (end 199.5 81.96) (width 0.2) (layer "F.Cu") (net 6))
 (segment (start 196.25 74.85) (end 196.25 79.3) (width 0.2) (layer "F.Cu") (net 6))
 (segment (start 199.39 81.85) (end 196.15 81.85) (width 0.2) (layer "F.Cu") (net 6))
 (segment (start 167.04 71.28) (end 165.36 72.96) (width 0.2) (layer "F.Cu") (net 6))
 (segment (start 197.75 70.43) (end 196.9 71.28) (width 0.2) (layer "F.Cu") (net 6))
 (segment (start 196.15 81.85) (end 196 82) (width 0.2) (layer "F.Cu") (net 6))
 (segment (start 197.75 70.43) (end 199.25 71.93) (width 0.2) (layer "F.Cu") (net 6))
 (segment (start 199.3 79.3) (end 199.5 79.5) (width 0.2) (layer "F.Cu") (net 6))
 (segment (start 196 83.92) (end 197.75 85.67) (width 0.2) (layer "F.Cu") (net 6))
 (segment (start 199.25 71.93) (end 199.25 74.2) (width 0.2) (layer "F.Cu") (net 6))
 (segment (start 142.745 57.965) (end 142.5 57.72) (width 0.2) (layer "F.Cu") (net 1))
 (segment (start 139.96 57.72) (end 139.96 60.26) (width 0.2) (layer "F.Cu") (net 1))
 (segment (start 196.02 56) (end 144.22 56) (width 0.2) (layer "F.Cu") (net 1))
 (segment (start 142.5 57.72) (end 142.5 60.26) (width 0.2) (layer "F.Cu") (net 1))
 (segment (start 199.49 75.51) (end 201.5 73.5) (width 0.2) (layer "F.Cu") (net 1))
 (segment (start 197.75 57.73) (end 196.02 56) (width 0.2) (layer "F.Cu") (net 1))
 (segment (start 144.22 56) (end 142.5 57.72) (width 0.2) (layer "F.Cu") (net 1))
 (segment (start 142.5 60.26) (end 112.8 60.26) (width 0.2) (layer "F.Cu") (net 1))
 (segment (start 112.8 60.26) (end 112.75 60.21) (width 0.2) (layer "F.Cu") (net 1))
 (segment (start 143.375 57.965) (end 142.745 57.965) (width 0.2) (layer "F.Cu") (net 1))
 (segment (start 201.5 61.48) (end 197.75 57.73) (width 0.2) (layer "F.Cu") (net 1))
 (segment (start 197.75 75.51) (end 199.49 75.51) (width 0.2) (layer "F.Cu") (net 1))
 (segment (start 201.5 73.5) (end 201.5 61.48) (width 0.2) (layer "F.Cu") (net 1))
 (segment (start 195.22 70.42) (end 197.75 67.89) (width 0.2) (layer "F.Cu") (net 5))
 (segment (start 165.36 70.42) (end 195.22 70.42) (width 0.2) (layer "F.Cu") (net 5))
 (segment (start 139.91 90.69) (end 139.96 90.74) (width 0.2) (layer "F.Cu") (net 23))
 (segment (start 142.5 90.74) (end 139.96 90.74) (width 0.2) (layer "F.Cu") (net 23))
 (segment (start 112.75 90.69) (end 139.91 90.69) (width 0.2) (layer "F.Cu") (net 23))
 (segment (start 139.90904 108.47) (end 139.95632 108.51728) (width 0.2) (layer "F.Cu") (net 30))
 (segment (start 112.75 108.47) (end 139.90904 108.47) (width 0.2) (layer "F.Cu") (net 30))
 (segment (start 142.49632 108.51728) (end 139.95632 108.51728) (width 0.2) (layer "F.Cu") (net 30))
 (segment (start 142.5 65.34) (end 112.8 65.34) (width 0.2) (layer "F.Cu") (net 13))
 (segment (start 112.8 65.34) (end 112.75 65.29) (width 0.2) (layer "F.Cu") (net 13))
 (segment (start 199.75 92.37) (end 197.62 94.5) (width 0.2) (layer "F.Cu") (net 9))
 (segment (start 197.75 83.13) (end 199.75 85.13) (width 0.2) (layer "F.Cu") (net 9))
 (segment (start 197.62 94.5) (end 162.75 94.5) (width 0.2) (layer "F.Cu") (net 9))
 (segment (start 162.75 94.5) (end 162.75 83.19) (width 0.2) (layer "F.Cu") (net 9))
 (segment (start 199.75 85.13) (end 199.75 92.37) (width 0.2) (layer "F.Cu") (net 9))
 (segment (start 162.75 83.19) (end 165.36 80.58) (width 0.2) (layer "F.Cu") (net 9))
 (segment (start 195.22 67.88) (end 197.75 65.35) (width 0.2) (layer "F.Cu") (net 4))
 (segment (start 165.36 67.88) (end 195.22 67.88) (width 0.2) (layer "F.Cu") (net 4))
 (segment (start 142.5 80.58) (end 139.96 80.58) (width 0.2) (layer "F.Cu") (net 19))
 (segment (start 112.8 80.58) (end 112.75 80.53) (width 0.2) (layer "F.Cu") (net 19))
 (segment (start 139.96 80.58) (end 112.8 80.58) (width 0.2) (layer "F.Cu") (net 19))
 (segment (start 142.5 83.12) (end 139.96 83.12) (width 0.2) (layer "F.Cu") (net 20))
 (segment (start 139.91 83.07) (end 139.96 83.12) (width 0.2) (layer "F.Cu") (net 20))
 (segment (start 112.75 83.07) (end 139.91 83.07) (width 0.2) (layer "F.Cu") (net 20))
 (segment (start 112.8 85.66) (end 112.75 85.61) (width 0.2) (layer "F.Cu") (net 21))
 (segment (start 142.5 85.66) (end 139.96 85.66) (width 0.2) (layer "F.Cu") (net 21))
 (segment (start 139.96 85.66) (end 112.8 85.66) (width 0.2) (layer "F.Cu") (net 21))
 (segment (start 112.75 93.23) (end 139.91 93.23) (width 0.2) (layer "F.Cu") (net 24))
 (segment (start 142.5 93.28) (end 139.96 93.28) (width 0.2) (layer "F.Cu") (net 24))
 (segment (start 139.91 93.23) (end 139.96 93.28) (width 0.2) (layer "F.Cu") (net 24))
 (segment (start 139.91 72.91) (end 139.96 72.96) (width 0.2) (layer "F.Cu") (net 16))
 (segment (start 142.5 72.96) (end 139.96 72.96) (width 0.2) (layer "F.Cu") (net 16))
 (segment (start 112.75 72.91) (end 139.91 72.91) (width 0.2) (layer "F.Cu") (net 16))
 (segment (start 165.25 62.69) (end 165.25 62.47) (width 0.2) (layer "F.Cu") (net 41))
 (segment (start 165.36 62.8) (end 165.36 62.4) (width 0.2) (layer "F.Cu") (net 41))
 (segment (start 195.25 72.97) (end 192.72 75.5) (width 0.2) (layer "F.Cu") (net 7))
 (segment (start 197.23 72.97) (end 197.75 72.97) (width 0.2) (layer "F.Cu") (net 7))
 (segment (start 197.75 72.97) (end 195.25 72.97) (width 0.2) (layer "F.Cu") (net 7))
 (segment (start 197.75 80.59) (end 195.25 80.59) (width 0.2) (layer "F.Cu") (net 7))
 (segment (start 195.25 80.59) (end 195.25 74.95) (width 0.2) (layer "F.Cu") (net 7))
 (segment (start 192.72 75.5) (end 165.36 75.5) (width 0.2) (layer "F.Cu") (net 7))
 (segment (start 195.25 74.95) (end 197.23 72.97) (width 0.2) (layer "F.Cu") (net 7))
 (segment (start 165.36 65.34) (end 195.22 65.34) (width 0.2) (layer "F.Cu") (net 3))
 (segment (start 195.22 65.34) (end 197.75 62.81) (width 0.2) (layer "F.Cu") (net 3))
 (segment (start 142.5 103.44) (end 139.96 103.44) (width 0.2) (layer "F.Cu") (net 28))
 (segment (start 139.96 103.44) (end 112.8 103.44) (width 0.2) (layer "F.Cu") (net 28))
 (segment (start 112.8 103.44) (end 112.75 103.39) (width 0.2) (layer "F.Cu") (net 28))
 (segment (start 112.75 77.99) (end 139.91 77.99) (width 0.2) (layer "F.Cu") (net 18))
 (segment (start 139.91 77.99) (end 139.96 78.04) (width 0.2) (layer "F.Cu") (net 18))
 (segment (start 142.5 78.04) (end 139.96 78.04) (width 0.2) (layer "F.Cu") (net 18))
 (segment (start 142.5 95.82) (end 139.96 95.82) (width 0.2) (layer "F.Cu") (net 25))
 (segment (start 139.91 95.77) (end 139.96 95.82) (width 0.2) (layer "F.Cu") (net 25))
 (segment (start 112.75 95.77) (end 139.91 95.77) (width 0.2) (layer "F.Cu") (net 25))
 (segment (start 112.8 75.5) (end 112.75 75.45) (width 0.2) (layer "F.Cu") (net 17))
 (segment (start 142.5 75.5) (end 139.96 75.5) (width 0.2) (layer "F.Cu") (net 17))
 (segment (start 139.96 75.5) (end 112.8 75.5) (width 0.2) (layer "F.Cu") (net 17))
 (segment (start 198.17 78.05) (end 198.25 77.97) (width 0.2) (layer "F.Cu") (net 8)))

